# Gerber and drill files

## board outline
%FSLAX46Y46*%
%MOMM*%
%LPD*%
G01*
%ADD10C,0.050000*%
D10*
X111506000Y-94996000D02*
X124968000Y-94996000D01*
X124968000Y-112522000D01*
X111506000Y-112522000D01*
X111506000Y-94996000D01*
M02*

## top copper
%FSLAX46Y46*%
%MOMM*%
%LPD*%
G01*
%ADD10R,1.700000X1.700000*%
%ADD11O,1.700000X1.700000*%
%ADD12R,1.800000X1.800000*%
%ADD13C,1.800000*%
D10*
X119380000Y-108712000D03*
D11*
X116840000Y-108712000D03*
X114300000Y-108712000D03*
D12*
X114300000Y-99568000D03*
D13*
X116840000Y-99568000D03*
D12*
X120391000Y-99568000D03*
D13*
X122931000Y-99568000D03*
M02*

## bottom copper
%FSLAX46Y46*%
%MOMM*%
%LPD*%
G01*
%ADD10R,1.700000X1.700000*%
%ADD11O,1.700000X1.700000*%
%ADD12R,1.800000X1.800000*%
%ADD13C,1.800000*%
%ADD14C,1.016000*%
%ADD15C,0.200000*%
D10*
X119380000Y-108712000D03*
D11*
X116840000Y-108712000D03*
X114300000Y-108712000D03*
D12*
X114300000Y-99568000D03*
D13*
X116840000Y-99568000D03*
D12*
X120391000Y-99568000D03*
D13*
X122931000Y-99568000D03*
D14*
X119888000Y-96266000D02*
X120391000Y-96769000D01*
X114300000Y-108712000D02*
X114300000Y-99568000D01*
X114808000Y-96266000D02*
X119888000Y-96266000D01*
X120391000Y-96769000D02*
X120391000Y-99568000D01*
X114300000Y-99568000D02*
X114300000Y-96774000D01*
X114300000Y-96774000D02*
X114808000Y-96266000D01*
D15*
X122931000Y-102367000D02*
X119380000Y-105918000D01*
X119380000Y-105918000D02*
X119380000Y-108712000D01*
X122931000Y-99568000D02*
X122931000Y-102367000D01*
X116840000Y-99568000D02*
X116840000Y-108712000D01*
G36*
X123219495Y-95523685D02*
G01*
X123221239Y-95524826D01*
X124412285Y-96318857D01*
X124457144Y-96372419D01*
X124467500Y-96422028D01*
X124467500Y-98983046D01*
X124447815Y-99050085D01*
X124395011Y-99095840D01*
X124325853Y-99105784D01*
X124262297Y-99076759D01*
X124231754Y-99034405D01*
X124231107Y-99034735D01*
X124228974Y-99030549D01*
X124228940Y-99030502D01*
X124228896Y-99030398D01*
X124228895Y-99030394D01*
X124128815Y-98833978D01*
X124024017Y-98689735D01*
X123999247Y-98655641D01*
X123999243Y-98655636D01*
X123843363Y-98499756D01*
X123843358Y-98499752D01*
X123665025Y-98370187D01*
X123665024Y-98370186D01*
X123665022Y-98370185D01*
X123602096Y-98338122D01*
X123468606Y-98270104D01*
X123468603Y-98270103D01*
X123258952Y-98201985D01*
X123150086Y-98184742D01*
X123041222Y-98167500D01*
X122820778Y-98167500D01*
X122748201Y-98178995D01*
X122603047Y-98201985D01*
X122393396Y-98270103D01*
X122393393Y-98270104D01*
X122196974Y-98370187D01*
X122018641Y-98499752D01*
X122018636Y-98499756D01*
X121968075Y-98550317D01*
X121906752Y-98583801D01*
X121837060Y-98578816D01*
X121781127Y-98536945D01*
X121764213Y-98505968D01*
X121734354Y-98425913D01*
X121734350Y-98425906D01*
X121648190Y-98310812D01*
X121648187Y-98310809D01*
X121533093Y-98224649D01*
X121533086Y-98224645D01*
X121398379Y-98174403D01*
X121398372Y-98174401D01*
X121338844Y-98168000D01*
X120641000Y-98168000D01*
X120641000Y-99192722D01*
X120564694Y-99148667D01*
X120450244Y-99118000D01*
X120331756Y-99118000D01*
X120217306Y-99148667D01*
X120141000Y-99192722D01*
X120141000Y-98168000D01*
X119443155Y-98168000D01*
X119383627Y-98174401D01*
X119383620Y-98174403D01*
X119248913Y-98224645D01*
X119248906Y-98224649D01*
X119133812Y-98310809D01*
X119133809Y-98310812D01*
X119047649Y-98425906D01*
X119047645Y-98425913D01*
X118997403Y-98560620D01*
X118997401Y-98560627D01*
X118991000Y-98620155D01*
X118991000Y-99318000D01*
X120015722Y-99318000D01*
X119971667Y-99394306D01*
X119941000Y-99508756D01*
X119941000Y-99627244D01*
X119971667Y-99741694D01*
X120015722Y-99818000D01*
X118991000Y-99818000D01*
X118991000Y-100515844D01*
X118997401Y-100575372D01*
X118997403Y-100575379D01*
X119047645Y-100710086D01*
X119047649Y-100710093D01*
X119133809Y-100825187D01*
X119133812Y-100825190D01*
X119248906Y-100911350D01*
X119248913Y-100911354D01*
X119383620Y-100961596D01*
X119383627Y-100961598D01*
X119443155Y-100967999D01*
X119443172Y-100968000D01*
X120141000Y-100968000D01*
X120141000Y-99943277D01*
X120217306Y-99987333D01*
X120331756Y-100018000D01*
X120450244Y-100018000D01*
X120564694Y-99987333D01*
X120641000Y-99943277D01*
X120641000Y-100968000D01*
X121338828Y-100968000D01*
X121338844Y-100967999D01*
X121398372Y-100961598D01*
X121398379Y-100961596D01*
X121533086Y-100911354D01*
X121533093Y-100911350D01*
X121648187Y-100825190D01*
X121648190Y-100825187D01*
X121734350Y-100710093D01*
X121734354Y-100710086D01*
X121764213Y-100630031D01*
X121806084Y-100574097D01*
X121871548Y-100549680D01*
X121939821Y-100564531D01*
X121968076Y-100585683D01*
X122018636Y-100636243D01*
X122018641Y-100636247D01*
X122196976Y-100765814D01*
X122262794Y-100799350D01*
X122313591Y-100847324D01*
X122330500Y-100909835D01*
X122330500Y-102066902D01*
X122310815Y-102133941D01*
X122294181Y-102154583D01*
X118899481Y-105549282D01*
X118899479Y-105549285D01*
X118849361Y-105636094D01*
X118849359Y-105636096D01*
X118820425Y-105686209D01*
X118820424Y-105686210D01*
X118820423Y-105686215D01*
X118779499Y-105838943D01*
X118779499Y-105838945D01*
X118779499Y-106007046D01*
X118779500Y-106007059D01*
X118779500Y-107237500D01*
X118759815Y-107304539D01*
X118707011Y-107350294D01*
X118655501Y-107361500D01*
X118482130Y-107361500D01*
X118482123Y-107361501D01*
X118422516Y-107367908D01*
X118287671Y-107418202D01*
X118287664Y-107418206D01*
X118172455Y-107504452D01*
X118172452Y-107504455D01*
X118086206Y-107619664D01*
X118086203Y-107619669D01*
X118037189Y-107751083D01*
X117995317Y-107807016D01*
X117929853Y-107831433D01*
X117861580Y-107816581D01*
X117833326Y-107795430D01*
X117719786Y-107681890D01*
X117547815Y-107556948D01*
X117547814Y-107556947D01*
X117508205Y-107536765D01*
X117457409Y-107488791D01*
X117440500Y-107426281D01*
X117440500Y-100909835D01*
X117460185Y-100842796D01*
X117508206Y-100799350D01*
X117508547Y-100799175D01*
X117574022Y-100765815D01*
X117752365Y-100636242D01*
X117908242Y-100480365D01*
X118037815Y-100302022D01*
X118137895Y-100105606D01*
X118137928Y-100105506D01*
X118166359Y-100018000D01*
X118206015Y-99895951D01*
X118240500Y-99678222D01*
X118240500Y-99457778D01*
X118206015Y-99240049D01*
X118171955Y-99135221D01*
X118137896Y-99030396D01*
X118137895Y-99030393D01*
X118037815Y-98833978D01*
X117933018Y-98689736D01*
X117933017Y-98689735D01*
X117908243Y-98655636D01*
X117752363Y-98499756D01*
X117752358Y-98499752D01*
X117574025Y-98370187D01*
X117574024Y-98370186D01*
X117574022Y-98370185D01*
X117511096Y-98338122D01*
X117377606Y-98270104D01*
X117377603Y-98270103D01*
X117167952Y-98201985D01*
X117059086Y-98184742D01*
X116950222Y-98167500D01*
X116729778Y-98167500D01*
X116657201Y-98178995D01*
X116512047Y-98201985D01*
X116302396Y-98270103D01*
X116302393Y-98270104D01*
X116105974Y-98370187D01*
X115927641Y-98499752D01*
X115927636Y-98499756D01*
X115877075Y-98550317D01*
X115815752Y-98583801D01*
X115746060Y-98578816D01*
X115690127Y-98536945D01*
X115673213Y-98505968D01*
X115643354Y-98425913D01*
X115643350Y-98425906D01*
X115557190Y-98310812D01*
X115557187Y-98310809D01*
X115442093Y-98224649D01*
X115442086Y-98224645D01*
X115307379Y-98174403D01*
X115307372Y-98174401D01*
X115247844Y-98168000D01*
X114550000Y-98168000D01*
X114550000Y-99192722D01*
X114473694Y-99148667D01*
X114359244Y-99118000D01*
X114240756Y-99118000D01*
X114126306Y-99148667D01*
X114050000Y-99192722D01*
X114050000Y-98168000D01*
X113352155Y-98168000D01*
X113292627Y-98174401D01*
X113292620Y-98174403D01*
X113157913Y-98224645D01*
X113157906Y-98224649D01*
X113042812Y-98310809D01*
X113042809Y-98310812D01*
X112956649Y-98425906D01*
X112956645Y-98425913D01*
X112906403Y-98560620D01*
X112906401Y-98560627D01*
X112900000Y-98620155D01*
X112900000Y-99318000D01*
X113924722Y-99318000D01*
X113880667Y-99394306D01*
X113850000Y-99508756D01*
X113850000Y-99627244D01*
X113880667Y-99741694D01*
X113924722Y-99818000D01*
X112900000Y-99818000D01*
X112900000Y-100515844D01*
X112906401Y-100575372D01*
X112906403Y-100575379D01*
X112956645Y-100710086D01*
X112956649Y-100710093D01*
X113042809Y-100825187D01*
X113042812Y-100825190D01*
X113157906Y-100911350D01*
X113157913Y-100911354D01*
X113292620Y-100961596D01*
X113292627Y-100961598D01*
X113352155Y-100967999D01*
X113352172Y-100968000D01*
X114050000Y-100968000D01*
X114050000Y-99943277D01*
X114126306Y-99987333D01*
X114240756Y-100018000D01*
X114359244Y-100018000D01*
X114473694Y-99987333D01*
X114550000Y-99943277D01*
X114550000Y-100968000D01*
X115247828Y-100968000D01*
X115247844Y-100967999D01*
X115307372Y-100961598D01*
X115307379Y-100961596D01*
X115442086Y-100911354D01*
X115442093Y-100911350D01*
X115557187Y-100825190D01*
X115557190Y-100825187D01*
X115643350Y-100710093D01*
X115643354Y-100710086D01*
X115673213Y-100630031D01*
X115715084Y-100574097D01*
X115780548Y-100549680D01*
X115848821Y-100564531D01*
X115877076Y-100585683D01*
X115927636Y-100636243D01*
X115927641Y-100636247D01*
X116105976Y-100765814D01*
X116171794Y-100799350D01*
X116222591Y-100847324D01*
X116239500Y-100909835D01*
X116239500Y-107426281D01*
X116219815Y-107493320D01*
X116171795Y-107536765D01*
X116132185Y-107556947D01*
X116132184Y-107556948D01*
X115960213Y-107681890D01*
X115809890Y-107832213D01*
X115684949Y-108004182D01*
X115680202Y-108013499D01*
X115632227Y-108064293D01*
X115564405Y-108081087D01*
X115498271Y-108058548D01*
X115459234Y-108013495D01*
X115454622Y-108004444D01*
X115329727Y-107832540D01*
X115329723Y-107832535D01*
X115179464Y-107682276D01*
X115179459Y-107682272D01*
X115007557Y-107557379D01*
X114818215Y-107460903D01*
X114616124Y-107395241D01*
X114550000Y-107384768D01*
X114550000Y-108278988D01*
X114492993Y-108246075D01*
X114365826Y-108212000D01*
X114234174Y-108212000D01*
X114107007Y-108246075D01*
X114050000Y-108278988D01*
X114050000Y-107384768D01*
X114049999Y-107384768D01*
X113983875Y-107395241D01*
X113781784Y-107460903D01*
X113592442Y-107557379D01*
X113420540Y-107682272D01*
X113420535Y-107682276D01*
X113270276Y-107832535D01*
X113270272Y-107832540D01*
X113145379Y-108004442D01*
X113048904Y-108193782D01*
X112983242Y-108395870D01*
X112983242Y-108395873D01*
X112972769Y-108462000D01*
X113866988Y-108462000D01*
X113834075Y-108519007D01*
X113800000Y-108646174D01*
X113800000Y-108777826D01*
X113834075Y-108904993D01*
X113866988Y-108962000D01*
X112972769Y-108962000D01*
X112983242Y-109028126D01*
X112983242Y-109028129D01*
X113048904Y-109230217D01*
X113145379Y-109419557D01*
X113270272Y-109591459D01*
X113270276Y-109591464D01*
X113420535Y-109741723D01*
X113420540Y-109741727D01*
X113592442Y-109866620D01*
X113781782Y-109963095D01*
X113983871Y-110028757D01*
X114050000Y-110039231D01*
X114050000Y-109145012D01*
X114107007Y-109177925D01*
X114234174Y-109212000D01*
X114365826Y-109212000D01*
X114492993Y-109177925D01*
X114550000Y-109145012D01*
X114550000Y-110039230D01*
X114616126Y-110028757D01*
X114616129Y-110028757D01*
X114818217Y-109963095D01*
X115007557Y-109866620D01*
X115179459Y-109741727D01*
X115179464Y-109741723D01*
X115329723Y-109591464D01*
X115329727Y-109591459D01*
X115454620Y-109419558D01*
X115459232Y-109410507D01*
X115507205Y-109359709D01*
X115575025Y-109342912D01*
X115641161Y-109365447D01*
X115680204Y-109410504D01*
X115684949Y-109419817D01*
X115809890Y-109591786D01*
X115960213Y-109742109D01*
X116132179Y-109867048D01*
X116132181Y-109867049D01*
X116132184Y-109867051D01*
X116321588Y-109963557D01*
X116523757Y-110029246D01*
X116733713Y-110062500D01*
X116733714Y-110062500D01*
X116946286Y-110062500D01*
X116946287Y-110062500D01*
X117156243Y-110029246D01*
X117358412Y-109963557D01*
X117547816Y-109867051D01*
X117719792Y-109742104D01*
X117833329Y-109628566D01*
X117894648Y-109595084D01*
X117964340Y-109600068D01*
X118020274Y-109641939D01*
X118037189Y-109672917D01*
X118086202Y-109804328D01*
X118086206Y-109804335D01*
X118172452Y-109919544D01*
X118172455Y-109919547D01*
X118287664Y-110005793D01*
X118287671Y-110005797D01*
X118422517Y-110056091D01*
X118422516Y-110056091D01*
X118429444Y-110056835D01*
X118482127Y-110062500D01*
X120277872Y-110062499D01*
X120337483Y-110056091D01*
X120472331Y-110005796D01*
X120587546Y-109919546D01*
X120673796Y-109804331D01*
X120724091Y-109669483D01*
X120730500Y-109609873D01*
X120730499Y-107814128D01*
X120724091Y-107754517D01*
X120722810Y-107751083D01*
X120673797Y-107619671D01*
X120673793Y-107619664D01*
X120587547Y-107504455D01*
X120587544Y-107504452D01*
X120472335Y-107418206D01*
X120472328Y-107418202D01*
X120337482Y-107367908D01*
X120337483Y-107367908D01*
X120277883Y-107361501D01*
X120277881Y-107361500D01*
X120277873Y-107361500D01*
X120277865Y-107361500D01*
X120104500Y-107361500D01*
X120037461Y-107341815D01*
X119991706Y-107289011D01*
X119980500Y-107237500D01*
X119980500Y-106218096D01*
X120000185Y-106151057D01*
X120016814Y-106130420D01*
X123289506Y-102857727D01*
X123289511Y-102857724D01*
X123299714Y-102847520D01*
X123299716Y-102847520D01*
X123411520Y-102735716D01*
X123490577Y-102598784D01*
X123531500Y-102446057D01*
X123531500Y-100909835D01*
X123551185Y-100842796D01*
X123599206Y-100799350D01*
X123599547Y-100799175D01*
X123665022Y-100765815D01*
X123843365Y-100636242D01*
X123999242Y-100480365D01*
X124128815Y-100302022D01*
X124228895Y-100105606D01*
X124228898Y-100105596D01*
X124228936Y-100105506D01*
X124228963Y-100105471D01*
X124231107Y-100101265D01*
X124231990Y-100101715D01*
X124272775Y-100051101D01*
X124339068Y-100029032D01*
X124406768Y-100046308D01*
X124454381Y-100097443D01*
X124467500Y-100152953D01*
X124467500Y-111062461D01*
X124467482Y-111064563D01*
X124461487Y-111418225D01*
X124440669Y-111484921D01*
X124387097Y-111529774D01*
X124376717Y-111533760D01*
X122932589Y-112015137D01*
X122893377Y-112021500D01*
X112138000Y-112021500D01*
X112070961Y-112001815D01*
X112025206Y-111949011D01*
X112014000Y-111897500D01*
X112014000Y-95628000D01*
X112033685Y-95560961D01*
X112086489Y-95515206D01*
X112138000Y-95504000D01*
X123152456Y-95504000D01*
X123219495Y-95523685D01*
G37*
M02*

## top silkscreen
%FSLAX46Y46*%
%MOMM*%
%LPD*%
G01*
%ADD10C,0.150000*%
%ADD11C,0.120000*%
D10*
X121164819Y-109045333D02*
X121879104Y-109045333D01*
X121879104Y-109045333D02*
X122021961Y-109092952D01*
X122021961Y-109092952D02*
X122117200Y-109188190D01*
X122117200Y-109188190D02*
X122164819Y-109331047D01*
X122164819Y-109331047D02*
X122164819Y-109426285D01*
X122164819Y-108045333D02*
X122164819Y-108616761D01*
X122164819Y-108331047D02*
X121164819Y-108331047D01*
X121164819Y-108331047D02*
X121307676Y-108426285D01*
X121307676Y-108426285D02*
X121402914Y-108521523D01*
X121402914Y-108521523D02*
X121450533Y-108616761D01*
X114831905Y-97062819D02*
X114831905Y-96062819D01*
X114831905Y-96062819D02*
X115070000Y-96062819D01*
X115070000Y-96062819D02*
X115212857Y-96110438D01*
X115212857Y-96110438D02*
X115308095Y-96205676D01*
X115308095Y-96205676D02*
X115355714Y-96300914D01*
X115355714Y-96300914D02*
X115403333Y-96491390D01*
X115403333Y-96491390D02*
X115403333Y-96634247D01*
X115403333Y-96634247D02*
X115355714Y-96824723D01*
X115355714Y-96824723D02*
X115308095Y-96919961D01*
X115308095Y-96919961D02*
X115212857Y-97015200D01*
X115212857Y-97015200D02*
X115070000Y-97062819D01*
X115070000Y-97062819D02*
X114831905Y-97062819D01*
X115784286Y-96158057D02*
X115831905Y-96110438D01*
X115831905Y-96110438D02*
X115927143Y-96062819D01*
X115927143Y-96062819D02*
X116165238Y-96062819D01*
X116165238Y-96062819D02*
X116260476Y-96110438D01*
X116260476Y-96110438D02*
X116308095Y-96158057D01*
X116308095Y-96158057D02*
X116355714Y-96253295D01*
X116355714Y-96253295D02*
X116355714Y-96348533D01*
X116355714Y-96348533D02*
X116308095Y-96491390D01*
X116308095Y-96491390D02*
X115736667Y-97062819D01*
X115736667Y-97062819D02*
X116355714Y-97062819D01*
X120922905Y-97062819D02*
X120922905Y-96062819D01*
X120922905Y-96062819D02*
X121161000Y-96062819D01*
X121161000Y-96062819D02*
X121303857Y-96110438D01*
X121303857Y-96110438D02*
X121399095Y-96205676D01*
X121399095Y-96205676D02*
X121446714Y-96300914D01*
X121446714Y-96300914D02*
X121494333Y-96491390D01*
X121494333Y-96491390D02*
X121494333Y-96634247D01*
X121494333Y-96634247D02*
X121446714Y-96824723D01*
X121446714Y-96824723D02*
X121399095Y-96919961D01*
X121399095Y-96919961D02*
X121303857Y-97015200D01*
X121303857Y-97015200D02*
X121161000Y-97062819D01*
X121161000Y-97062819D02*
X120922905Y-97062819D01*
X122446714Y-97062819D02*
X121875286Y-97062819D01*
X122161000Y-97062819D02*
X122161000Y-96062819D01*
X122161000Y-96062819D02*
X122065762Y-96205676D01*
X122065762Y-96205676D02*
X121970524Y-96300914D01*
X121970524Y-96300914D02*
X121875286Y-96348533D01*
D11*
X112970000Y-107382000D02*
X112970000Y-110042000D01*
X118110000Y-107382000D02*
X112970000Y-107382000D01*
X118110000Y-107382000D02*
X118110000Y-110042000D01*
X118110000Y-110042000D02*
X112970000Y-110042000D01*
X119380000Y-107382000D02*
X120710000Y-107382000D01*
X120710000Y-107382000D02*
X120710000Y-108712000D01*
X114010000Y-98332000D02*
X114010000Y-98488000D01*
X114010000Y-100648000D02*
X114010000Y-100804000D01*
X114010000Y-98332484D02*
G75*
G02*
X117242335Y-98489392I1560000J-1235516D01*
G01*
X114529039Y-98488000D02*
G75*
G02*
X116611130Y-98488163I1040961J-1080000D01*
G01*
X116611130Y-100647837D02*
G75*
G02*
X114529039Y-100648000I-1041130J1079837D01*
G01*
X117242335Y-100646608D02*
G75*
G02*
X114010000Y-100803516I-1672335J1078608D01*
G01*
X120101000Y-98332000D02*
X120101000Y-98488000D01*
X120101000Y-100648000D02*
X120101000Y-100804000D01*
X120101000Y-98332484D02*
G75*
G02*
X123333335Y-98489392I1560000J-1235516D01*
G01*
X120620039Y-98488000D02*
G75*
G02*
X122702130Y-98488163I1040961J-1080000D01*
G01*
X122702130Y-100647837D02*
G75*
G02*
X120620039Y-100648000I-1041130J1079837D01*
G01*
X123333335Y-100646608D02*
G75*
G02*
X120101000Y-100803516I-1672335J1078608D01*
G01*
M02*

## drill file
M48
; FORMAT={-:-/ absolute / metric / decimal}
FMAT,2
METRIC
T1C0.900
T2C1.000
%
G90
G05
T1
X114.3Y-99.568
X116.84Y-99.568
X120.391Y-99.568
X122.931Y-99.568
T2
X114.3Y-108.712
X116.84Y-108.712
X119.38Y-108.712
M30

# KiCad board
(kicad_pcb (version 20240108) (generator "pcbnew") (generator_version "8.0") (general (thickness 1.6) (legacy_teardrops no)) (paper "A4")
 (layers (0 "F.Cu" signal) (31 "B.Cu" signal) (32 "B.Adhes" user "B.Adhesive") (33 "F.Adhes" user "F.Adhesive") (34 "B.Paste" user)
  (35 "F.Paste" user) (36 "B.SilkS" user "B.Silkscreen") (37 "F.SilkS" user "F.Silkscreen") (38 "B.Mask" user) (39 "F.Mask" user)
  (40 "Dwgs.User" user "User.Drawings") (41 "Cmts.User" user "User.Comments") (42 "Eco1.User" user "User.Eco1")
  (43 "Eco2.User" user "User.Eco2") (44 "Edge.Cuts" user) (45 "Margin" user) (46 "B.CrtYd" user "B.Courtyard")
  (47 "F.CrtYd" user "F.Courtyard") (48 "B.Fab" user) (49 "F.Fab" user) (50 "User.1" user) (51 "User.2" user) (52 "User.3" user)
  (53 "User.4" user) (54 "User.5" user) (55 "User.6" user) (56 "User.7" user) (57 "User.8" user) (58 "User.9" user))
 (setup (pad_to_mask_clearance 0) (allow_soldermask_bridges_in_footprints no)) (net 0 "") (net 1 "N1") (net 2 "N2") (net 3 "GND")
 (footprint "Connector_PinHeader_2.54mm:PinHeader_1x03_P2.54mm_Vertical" (layer "F.Cu") (at 119.38 108.712 -90)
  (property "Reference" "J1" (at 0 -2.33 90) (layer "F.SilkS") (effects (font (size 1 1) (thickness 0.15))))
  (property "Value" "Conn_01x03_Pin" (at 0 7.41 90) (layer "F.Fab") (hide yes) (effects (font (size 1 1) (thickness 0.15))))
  (fp_line (start -1.33 6.41) (end 1.33 6.41) (stroke (width 0.12) (type solid)) (layer "F.SilkS"))
  (fp_line (start -1.33 1.27) (end -1.33 6.41) (stroke (width 0.12) (type solid)) (layer "F.SilkS"))
  (fp_line (start -1.33 1.27) (end 1.33 1.27) (stroke (width 0.12) (type solid)) (layer "F.SilkS"))
  (fp_line (start 1.33 1.27) (end 1.33 6.41) (stroke (width 0.12) (type solid)) (layer "F.SilkS"))
  (fp_line (start -1.33 0) (end -1.33 -1.33) (stroke (width 0.12) (type solid)) (layer "F.SilkS"))
  (fp_line (start -1.33 -1.33) (end 0 -1.33) (stroke (width 0.12) (type solid)) (layer "F.SilkS"))
  (pad "1" thru_hole rect (at 0 0 270) (size 1.7 1.7) (drill 1) (layers "*.Cu" "*.Mask") (remove_unused_layers no) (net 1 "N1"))
  (pad "2" thru_hole oval (at 0 2.54 270) (size 1.7 1.7) (drill 1) (layers "*.Cu" "*.Mask") (remove_unused_layers no) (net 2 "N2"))
  (pad "3" thru_hole oval (at 0 5.08 270) (size 1.7 1.7) (drill 1) (layers "*.Cu" "*.Mask") (remove_unused_layers no) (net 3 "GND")))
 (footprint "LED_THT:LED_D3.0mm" (layer "F.Cu") (at 114.3 99.568)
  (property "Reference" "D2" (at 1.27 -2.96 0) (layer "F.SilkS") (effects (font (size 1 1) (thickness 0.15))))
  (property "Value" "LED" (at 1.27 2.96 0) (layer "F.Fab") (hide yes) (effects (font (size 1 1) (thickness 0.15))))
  (fp_line (start -0.29 -1.236) (end -0.29 -1.08) (stroke (width 0.12) (type solid)) (layer "F.SilkS"))
  (fp_line (start -0.29 1.08) (end -0.29 1.236) (stroke (width 0.12) (type solid)) (layer "F.SilkS"))
  (fp_arc (start -0.29 -1.235516) (mid 1.366487 -1.987659) (end 2.942335 -1.078608) (stroke (width 0.12) (type solid)) (layer "F.SilkS"))
  (fp_arc (start 0.229039 -1.08) (mid 1.270117 -1.5) (end 2.31113 -1.079837) (stroke (width 0.12) (type solid)) (layer "F.SilkS"))
  (fp_arc (start 2.31113 1.079837) (mid 1.270117 1.5) (end 0.229039 1.08) (stroke (width 0.12) (type solid)) (layer "F.SilkS"))
  (fp_arc (start 2.942335 1.078608) (mid 1.366487 1.987659) (end -0.29 1.235516) (stroke (width 0.12) (type solid)) (layer "F.SilkS"))
  (pad "1" thru_hole rect (at 0 0) (size 1.8 1.8) (drill 0.9) (layers "*.Cu" "*.Mask") (remove_unused_layers no) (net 3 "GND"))
  (pad "2" thru_hole circle (at 2.54 0) (size 1.8 1.8) (drill 0.9) (layers "*.Cu" "*.Mask") (remove_unused_layers no) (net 2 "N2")))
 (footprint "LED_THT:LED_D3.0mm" (layer "F.Cu") (at 120.391 99.568)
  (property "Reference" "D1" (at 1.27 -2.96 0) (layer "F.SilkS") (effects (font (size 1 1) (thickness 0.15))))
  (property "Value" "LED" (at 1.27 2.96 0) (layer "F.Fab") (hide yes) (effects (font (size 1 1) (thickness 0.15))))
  (fp_line (start -0.29 -1.236) (end -0.29 -1.08) (stroke (width 0.12) (type solid)) (layer "F.SilkS"))
  (fp_line (start -0.29 1.08) (end -0.29 1.236) (stroke (width 0.12) (type solid)) (layer "F.SilkS"))
  (fp_arc (start -0.29 -1.235516) (mid 1.366487 -1.987659) (end 2.942335 -1.078608) (stroke (width 0.12) (type solid)) (layer "F.SilkS"))
  (fp_arc (start 0.229039 -1.08) (mid 1.270117 -1.5) (end 2.31113 -1.079837) (stroke (width 0.12) (type solid)) (layer "F.SilkS"))
  (fp_arc (start 2.31113 1.079837) (mid 1.270117 1.5) (end 0.229039 1.08) (stroke (width 0.12) (type solid)) (layer "F.SilkS"))
  (fp_arc (start 2.942335 1.078608) (mid 1.366487 1.987659) (end -0.29 1.235516) (stroke (width 0.12) (type solid)) (layer "F.SilkS"))
  (pad "1" thru_hole rect (at 0 0) (size 1.8 1.8) (drill 0.9) (layers "*.Cu" "*.Mask") (remove_unused_layers no) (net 3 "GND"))
  (pad "2" thru_hole circle (at 2.54 0) (size 1.8 1.8) (drill 0.9) (layers "*.Cu" "*.Mask") (remove_unused_layers no) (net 1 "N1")))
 (gr_rect (start 111.506 94.996) (end 124.968 112.522) (stroke (width 0.05) (type default)) (fill none) (layer "Edge.Cuts"))
 (segment (start 119.888 96.266) (end 120.391 96.769) (width 1.016) (layer "B.Cu") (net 3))
 (segment (start 114.3 108.712) (end 114.3 99.568) (width 1.016) (layer "B.Cu") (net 3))
 (segment (start 114.808 96.266) (end 119.888 96.266) (width 1.016) (layer "B.Cu") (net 3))
 (segment (start 120.391 96.769) (end 120.391 99.568) (width 1.016) (layer "B.Cu") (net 3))
 (segment (start 114.3 99.568) (end 114.3 96.774) (width 1.016) (layer "B.Cu") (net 3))
 (segment (start 114.3 96.774) (end 114.808 96.266) (width 1.016) (layer "B.Cu") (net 3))
 (segment (start 122.931 102.367) (end 119.38 105.918) (width 0.2) (layer "B.Cu") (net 1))
 (segment (start 119.38 105.918) (end 119.38 108.712) (width 0.2) (layer "B.Cu") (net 1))
 (segment (start 122.931 99.568) (end 122.931 102.367) (width 0.2) (layer "B.Cu") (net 1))
 (segment (start 116.84 99.568) (end 116.84 108.712) (width 0.2) (layer "B.Cu") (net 2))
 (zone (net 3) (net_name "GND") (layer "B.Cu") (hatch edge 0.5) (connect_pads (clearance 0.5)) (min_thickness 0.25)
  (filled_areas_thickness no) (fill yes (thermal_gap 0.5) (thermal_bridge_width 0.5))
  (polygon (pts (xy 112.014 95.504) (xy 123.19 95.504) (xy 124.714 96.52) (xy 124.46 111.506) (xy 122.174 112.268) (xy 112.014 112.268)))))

